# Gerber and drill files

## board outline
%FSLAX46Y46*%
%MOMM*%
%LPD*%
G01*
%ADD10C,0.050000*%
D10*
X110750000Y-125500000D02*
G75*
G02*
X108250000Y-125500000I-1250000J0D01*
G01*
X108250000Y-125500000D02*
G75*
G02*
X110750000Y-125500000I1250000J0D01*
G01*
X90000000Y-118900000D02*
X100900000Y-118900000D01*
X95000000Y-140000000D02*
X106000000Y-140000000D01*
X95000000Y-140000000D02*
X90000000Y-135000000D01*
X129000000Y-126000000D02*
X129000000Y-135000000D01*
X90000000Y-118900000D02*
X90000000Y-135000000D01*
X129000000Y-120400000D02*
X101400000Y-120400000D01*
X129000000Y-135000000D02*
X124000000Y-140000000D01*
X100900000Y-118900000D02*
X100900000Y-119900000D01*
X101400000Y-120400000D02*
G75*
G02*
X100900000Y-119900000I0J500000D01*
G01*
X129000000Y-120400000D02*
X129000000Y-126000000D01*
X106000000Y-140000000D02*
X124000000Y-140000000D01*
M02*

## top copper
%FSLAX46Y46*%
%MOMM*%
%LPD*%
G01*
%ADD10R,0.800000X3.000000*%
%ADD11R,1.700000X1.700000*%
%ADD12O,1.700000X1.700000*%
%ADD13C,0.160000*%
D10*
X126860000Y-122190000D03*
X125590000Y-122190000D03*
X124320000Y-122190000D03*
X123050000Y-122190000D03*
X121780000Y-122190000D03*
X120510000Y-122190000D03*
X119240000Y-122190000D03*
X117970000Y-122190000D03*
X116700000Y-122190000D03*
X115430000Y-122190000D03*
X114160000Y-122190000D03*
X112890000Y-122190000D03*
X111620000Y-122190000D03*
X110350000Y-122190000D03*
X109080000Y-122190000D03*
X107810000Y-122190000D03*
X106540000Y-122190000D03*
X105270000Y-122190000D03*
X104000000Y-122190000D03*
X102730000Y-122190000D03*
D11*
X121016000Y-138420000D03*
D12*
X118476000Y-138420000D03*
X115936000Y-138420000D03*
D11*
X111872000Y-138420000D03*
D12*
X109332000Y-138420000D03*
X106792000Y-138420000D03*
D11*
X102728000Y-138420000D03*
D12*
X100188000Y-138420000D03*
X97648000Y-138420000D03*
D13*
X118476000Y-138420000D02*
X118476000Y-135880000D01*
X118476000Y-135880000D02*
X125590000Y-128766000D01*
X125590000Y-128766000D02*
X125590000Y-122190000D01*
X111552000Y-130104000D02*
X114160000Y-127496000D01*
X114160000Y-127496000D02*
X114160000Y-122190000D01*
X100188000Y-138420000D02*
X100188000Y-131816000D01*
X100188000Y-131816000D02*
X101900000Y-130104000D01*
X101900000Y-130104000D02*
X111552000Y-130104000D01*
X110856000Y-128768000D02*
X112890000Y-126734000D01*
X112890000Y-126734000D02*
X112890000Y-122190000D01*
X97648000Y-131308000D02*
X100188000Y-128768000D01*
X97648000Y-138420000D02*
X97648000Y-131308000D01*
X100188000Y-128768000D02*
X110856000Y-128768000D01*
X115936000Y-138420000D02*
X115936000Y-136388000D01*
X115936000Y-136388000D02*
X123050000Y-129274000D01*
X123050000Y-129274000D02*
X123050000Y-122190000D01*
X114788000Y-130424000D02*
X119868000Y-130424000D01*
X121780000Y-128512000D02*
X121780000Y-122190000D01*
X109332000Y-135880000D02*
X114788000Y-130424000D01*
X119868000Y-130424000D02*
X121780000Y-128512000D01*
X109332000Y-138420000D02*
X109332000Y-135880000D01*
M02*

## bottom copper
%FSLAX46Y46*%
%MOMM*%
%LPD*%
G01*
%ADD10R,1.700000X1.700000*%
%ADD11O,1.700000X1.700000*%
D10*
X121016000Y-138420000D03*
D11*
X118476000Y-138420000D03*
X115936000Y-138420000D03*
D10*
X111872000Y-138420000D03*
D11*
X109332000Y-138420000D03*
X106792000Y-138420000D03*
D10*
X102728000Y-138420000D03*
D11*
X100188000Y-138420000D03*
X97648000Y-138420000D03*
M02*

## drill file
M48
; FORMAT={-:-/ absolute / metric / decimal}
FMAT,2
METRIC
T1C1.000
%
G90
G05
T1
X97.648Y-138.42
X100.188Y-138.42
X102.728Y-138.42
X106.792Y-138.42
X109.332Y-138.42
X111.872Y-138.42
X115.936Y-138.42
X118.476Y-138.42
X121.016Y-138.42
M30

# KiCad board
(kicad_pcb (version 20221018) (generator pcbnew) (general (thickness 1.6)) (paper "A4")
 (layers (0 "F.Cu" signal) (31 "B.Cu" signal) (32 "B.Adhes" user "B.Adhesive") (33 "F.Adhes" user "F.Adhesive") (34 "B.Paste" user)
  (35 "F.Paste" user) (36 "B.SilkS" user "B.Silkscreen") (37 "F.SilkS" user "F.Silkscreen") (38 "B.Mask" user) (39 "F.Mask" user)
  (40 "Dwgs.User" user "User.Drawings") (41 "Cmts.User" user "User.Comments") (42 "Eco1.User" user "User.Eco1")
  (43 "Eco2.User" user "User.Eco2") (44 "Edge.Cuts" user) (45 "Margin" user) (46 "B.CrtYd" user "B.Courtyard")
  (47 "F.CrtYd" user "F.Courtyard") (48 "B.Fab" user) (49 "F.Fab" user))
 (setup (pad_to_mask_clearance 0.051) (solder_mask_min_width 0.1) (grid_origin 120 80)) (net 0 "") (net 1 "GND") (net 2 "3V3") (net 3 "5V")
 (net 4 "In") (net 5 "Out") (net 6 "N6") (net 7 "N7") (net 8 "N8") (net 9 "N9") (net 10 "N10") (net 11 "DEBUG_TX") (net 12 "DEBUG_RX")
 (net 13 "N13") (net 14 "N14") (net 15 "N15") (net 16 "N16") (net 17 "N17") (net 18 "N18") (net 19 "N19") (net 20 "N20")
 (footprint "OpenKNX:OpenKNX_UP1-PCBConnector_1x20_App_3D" (layer "F.Cu") (at 126.86 122.19 180)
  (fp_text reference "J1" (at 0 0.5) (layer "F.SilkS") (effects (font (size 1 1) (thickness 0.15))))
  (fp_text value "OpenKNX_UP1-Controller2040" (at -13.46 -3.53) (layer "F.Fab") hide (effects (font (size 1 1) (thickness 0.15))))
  (pad "1" smd rect (at 0 0 270) (size 3 0.8) (layers "F.Cu" "F.Paste" "F.Mask") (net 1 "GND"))
  (pad "2" smd rect (at 1.27 0 270) (size 3 0.8) (layers "F.Cu" "F.Paste" "F.Mask") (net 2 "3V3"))
  (pad "3" smd rect (at 2.54 0 270) (size 3 0.8) (layers "F.Cu" "F.Paste" "F.Mask") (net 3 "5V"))
  (pad "4" smd rect (at 3.81 0 270) (size 3 0.8) (layers "F.Cu" "F.Paste" "F.Mask") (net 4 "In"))
  (pad "5" smd rect (at 5.08 0 270) (size 3 0.8) (layers "F.Cu" "F.Paste" "F.Mask") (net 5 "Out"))
  (pad "6" smd rect (at 6.35 0 270) (size 3 0.8) (layers "F.Cu" "F.Paste" "F.Mask") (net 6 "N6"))
  (pad "7" smd rect (at 7.62 0 270) (size 3 0.8) (layers "F.Cu" "F.Paste" "F.Mask") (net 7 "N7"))
  (pad "8" smd rect (at 8.89 0 270) (size 3 0.8) (layers "F.Cu" "F.Paste" "F.Mask") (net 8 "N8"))
  (pad "9" smd rect (at 10.16 0 270) (size 3 0.8) (layers "F.Cu" "F.Paste" "F.Mask") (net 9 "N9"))
  (pad "10" smd rect (at 11.43 0 270) (size 3 0.8) (layers "F.Cu" "F.Paste" "F.Mask") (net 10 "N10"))
  (pad "11" smd rect (at 12.7 0 270) (size 3 0.8) (layers "F.Cu" "F.Paste" "F.Mask") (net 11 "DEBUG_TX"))
  (pad "12" smd rect (at 13.97 0 270) (size 3 0.8) (layers "F.Cu" "F.Paste" "F.Mask") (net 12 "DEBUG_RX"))
  (pad "13" smd rect (at 15.24 0 270) (size 3 0.8) (layers "F.Cu" "F.Paste" "F.Mask") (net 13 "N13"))
  (pad "14" smd rect (at 16.51 0 270) (size 3 0.8) (layers "F.Cu" "F.Paste" "F.Mask") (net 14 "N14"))
  (pad "15" smd rect (at 17.78 0 270) (size 3 0.8) (layers "F.Cu" "F.Paste" "F.Mask") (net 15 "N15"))
  (pad "16" smd rect (at 19.05 0 270) (size 3 0.8) (layers "F.Cu" "F.Paste" "F.Mask") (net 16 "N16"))
  (pad "17" smd rect (at 20.32 0 270) (size 3 0.8) (layers "F.Cu" "F.Paste" "F.Mask") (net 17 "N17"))
  (pad "18" smd rect (at 21.59 0 270) (size 3 0.8) (layers "F.Cu" "F.Paste" "F.Mask") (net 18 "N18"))
  (pad "19" smd rect (at 22.86 0 270) (size 3 0.8) (layers "F.Cu" "F.Paste" "F.Mask") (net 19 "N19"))
  (pad "20" smd rect (at 24.13 0 270) (size 3 0.8) (layers "F.Cu" "F.Paste" "F.Mask") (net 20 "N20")))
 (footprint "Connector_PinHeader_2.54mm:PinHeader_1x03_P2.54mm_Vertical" (layer "F.Cu") (at 121.016 138.42 -90)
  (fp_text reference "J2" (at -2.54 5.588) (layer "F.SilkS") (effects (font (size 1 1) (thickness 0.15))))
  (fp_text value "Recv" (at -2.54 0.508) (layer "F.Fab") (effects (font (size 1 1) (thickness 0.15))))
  (pad "1" thru_hole rect (at 0 0 270) (size 1.7 1.7) (drill 1) (layers "*.Cu" "*.Mask") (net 1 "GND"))
  (pad "2" thru_hole oval (at 0 2.54 270) (size 1.7 1.7) (drill 1) (layers "*.Cu" "*.Mask") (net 2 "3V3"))
  (pad "3" thru_hole oval (at 0 5.08 270) (size 1.7 1.7) (drill 1) (layers "*.Cu" "*.Mask") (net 4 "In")))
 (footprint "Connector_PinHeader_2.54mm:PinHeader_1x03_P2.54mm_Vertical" (layer "F.Cu") (at 111.872 138.42 -90)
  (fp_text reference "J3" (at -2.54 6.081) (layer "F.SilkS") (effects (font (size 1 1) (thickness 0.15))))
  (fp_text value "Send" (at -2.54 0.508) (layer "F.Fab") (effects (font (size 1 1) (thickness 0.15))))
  (pad "1" thru_hole rect (at 0 0 270) (size 1.7 1.7) (drill 1) (layers "*.Cu" "*.Mask") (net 1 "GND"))
  (pad "2" thru_hole oval (at 0 2.54 270) (size 1.7 1.7) (drill 1) (layers "*.Cu" "*.Mask") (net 5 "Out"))
  (pad "3" thru_hole oval (at 0 5.08 270) (size 1.7 1.7) (drill 1) (layers "*.Cu" "*.Mask") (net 1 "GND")))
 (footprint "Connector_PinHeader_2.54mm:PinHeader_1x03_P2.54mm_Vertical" (layer "F.Cu") (at 102.728 138.42 -90)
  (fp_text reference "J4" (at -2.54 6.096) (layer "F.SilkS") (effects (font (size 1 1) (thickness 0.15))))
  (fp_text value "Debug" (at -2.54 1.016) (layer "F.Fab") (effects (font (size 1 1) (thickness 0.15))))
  (pad "1" thru_hole rect (at 0 0 270) (size 1.7 1.7) (drill 1) (layers "*.Cu" "*.Mask") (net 1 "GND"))
  (pad "2" thru_hole oval (at 0 2.54 270) (size 1.7 1.7) (drill 1) (layers "*.Cu" "*.Mask") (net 11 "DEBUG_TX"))
  (pad "3" thru_hole oval (at 0 5.08 270) (size 1.7 1.7) (drill 1) (layers "*.Cu" "*.Mask") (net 12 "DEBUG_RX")))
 (gr_circle (center 109.5 125.5) (end 109.5 124.25) (stroke (width 0.05) (type solid)) (fill none) (layer "Edge.Cuts"))
 (gr_line (start 90 118.9) (end 100.9 118.9) (stroke (width 0.05) (type solid)) (layer "Edge.Cuts"))
 (gr_line (start 95 140) (end 106 140) (stroke (width 0.05) (type solid)) (layer "Edge.Cuts"))
 (gr_line (start 95 140) (end 90 135) (stroke (width 0.05) (type solid)) (layer "Edge.Cuts"))
 (gr_line (start 129 126) (end 129 135) (stroke (width 0.05) (type solid)) (layer "Edge.Cuts"))
 (gr_line (start 90 118.9) (end 90 135) (stroke (width 0.05) (type solid)) (layer "Edge.Cuts"))
 (gr_line (start 129 120.4) (end 101.4 120.4) (stroke (width 0.05) (type solid)) (layer "Edge.Cuts"))
 (gr_line (start 129 135) (end 124 140) (stroke (width 0.05) (type solid)) (layer "Edge.Cuts"))
 (gr_line (start 100.9 118.9) (end 100.9 119.9) (stroke (width 0.05) (type solid)) (layer "Edge.Cuts"))
 (gr_arc (start 101.4 120.4) (mid 101.046447 120.253553) (end 100.9 119.9) (stroke (width 0.05) (type solid)) (layer "Edge.Cuts"))
 (gr_line (start 129 120.4) (end 129 126) (stroke (width 0.05) (type solid)) (layer "Edge.Cuts"))
 (gr_line (start 106 140) (end 124 140) (stroke (width 0.05) (type solid)) (layer "Edge.Cuts"))
 (segment (start 118.476 138.42) (end 118.476 135.88) (width 0.16) (layer "F.Cu") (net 2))
 (segment (start 118.476 135.88) (end 125.59 128.766) (width 0.16) (layer "F.Cu") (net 2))
 (segment (start 125.59 128.766) (end 125.59 122.19) (width 0.16) (layer "F.Cu") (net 2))
 (segment (start 111.552 130.104) (end 114.16 127.496) (width 0.16) (layer "F.Cu") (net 11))
 (segment (start 114.16 127.496) (end 114.16 122.19) (width 0.16) (layer "F.Cu") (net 11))
 (segment (start 100.188 138.42) (end 100.188 131.816) (width 0.16) (layer "F.Cu") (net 11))
 (segment (start 100.188 131.816) (end 101.9 130.104) (width 0.16) (layer "F.Cu") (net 11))
 (segment (start 101.9 130.104) (end 111.552 130.104) (width 0.16) (layer "F.Cu") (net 11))
 (segment (start 110.856 128.768) (end 112.89 126.734) (width 0.16) (layer "F.Cu") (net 12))
 (segment (start 112.89 126.734) (end 112.89 122.19) (width 0.16) (layer "F.Cu") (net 12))
 (segment (start 97.648 131.308) (end 100.188 128.768) (width 0.16) (layer "F.Cu") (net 12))
 (segment (start 97.648 138.42) (end 97.648 131.308) (width 0.16) (layer "F.Cu") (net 12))
 (segment (start 100.188 128.768) (end 110.856 128.768) (width 0.16) (layer "F.Cu") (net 12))
 (segment (start 115.936 138.42) (end 115.936 136.388) (width 0.16) (layer "F.Cu") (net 4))
 (segment (start 115.936 136.388) (end 123.05 129.274) (width 0.16) (layer "F.Cu") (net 4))
 (segment (start 123.05 129.274) (end 123.05 122.19) (width 0.16) (layer "F.Cu") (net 4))
 (segment (start 114.788 130.424) (end 119.868 130.424) (width 0.16) (layer "F.Cu") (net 5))
 (segment (start 121.78 128.512) (end 121.78 122.19) (width 0.16) (layer "F.Cu") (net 5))
 (segment (start 109.332 135.88) (end 114.788 130.424) (width 0.16) (layer "F.Cu") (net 5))
 (segment (start 119.868 130.424) (end 121.78 128.512) (width 0.16) (layer "F.Cu") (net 5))
 (segment (start 109.332 138.42) (end 109.332 135.88) (width 0.16) (layer "F.Cu") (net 5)))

